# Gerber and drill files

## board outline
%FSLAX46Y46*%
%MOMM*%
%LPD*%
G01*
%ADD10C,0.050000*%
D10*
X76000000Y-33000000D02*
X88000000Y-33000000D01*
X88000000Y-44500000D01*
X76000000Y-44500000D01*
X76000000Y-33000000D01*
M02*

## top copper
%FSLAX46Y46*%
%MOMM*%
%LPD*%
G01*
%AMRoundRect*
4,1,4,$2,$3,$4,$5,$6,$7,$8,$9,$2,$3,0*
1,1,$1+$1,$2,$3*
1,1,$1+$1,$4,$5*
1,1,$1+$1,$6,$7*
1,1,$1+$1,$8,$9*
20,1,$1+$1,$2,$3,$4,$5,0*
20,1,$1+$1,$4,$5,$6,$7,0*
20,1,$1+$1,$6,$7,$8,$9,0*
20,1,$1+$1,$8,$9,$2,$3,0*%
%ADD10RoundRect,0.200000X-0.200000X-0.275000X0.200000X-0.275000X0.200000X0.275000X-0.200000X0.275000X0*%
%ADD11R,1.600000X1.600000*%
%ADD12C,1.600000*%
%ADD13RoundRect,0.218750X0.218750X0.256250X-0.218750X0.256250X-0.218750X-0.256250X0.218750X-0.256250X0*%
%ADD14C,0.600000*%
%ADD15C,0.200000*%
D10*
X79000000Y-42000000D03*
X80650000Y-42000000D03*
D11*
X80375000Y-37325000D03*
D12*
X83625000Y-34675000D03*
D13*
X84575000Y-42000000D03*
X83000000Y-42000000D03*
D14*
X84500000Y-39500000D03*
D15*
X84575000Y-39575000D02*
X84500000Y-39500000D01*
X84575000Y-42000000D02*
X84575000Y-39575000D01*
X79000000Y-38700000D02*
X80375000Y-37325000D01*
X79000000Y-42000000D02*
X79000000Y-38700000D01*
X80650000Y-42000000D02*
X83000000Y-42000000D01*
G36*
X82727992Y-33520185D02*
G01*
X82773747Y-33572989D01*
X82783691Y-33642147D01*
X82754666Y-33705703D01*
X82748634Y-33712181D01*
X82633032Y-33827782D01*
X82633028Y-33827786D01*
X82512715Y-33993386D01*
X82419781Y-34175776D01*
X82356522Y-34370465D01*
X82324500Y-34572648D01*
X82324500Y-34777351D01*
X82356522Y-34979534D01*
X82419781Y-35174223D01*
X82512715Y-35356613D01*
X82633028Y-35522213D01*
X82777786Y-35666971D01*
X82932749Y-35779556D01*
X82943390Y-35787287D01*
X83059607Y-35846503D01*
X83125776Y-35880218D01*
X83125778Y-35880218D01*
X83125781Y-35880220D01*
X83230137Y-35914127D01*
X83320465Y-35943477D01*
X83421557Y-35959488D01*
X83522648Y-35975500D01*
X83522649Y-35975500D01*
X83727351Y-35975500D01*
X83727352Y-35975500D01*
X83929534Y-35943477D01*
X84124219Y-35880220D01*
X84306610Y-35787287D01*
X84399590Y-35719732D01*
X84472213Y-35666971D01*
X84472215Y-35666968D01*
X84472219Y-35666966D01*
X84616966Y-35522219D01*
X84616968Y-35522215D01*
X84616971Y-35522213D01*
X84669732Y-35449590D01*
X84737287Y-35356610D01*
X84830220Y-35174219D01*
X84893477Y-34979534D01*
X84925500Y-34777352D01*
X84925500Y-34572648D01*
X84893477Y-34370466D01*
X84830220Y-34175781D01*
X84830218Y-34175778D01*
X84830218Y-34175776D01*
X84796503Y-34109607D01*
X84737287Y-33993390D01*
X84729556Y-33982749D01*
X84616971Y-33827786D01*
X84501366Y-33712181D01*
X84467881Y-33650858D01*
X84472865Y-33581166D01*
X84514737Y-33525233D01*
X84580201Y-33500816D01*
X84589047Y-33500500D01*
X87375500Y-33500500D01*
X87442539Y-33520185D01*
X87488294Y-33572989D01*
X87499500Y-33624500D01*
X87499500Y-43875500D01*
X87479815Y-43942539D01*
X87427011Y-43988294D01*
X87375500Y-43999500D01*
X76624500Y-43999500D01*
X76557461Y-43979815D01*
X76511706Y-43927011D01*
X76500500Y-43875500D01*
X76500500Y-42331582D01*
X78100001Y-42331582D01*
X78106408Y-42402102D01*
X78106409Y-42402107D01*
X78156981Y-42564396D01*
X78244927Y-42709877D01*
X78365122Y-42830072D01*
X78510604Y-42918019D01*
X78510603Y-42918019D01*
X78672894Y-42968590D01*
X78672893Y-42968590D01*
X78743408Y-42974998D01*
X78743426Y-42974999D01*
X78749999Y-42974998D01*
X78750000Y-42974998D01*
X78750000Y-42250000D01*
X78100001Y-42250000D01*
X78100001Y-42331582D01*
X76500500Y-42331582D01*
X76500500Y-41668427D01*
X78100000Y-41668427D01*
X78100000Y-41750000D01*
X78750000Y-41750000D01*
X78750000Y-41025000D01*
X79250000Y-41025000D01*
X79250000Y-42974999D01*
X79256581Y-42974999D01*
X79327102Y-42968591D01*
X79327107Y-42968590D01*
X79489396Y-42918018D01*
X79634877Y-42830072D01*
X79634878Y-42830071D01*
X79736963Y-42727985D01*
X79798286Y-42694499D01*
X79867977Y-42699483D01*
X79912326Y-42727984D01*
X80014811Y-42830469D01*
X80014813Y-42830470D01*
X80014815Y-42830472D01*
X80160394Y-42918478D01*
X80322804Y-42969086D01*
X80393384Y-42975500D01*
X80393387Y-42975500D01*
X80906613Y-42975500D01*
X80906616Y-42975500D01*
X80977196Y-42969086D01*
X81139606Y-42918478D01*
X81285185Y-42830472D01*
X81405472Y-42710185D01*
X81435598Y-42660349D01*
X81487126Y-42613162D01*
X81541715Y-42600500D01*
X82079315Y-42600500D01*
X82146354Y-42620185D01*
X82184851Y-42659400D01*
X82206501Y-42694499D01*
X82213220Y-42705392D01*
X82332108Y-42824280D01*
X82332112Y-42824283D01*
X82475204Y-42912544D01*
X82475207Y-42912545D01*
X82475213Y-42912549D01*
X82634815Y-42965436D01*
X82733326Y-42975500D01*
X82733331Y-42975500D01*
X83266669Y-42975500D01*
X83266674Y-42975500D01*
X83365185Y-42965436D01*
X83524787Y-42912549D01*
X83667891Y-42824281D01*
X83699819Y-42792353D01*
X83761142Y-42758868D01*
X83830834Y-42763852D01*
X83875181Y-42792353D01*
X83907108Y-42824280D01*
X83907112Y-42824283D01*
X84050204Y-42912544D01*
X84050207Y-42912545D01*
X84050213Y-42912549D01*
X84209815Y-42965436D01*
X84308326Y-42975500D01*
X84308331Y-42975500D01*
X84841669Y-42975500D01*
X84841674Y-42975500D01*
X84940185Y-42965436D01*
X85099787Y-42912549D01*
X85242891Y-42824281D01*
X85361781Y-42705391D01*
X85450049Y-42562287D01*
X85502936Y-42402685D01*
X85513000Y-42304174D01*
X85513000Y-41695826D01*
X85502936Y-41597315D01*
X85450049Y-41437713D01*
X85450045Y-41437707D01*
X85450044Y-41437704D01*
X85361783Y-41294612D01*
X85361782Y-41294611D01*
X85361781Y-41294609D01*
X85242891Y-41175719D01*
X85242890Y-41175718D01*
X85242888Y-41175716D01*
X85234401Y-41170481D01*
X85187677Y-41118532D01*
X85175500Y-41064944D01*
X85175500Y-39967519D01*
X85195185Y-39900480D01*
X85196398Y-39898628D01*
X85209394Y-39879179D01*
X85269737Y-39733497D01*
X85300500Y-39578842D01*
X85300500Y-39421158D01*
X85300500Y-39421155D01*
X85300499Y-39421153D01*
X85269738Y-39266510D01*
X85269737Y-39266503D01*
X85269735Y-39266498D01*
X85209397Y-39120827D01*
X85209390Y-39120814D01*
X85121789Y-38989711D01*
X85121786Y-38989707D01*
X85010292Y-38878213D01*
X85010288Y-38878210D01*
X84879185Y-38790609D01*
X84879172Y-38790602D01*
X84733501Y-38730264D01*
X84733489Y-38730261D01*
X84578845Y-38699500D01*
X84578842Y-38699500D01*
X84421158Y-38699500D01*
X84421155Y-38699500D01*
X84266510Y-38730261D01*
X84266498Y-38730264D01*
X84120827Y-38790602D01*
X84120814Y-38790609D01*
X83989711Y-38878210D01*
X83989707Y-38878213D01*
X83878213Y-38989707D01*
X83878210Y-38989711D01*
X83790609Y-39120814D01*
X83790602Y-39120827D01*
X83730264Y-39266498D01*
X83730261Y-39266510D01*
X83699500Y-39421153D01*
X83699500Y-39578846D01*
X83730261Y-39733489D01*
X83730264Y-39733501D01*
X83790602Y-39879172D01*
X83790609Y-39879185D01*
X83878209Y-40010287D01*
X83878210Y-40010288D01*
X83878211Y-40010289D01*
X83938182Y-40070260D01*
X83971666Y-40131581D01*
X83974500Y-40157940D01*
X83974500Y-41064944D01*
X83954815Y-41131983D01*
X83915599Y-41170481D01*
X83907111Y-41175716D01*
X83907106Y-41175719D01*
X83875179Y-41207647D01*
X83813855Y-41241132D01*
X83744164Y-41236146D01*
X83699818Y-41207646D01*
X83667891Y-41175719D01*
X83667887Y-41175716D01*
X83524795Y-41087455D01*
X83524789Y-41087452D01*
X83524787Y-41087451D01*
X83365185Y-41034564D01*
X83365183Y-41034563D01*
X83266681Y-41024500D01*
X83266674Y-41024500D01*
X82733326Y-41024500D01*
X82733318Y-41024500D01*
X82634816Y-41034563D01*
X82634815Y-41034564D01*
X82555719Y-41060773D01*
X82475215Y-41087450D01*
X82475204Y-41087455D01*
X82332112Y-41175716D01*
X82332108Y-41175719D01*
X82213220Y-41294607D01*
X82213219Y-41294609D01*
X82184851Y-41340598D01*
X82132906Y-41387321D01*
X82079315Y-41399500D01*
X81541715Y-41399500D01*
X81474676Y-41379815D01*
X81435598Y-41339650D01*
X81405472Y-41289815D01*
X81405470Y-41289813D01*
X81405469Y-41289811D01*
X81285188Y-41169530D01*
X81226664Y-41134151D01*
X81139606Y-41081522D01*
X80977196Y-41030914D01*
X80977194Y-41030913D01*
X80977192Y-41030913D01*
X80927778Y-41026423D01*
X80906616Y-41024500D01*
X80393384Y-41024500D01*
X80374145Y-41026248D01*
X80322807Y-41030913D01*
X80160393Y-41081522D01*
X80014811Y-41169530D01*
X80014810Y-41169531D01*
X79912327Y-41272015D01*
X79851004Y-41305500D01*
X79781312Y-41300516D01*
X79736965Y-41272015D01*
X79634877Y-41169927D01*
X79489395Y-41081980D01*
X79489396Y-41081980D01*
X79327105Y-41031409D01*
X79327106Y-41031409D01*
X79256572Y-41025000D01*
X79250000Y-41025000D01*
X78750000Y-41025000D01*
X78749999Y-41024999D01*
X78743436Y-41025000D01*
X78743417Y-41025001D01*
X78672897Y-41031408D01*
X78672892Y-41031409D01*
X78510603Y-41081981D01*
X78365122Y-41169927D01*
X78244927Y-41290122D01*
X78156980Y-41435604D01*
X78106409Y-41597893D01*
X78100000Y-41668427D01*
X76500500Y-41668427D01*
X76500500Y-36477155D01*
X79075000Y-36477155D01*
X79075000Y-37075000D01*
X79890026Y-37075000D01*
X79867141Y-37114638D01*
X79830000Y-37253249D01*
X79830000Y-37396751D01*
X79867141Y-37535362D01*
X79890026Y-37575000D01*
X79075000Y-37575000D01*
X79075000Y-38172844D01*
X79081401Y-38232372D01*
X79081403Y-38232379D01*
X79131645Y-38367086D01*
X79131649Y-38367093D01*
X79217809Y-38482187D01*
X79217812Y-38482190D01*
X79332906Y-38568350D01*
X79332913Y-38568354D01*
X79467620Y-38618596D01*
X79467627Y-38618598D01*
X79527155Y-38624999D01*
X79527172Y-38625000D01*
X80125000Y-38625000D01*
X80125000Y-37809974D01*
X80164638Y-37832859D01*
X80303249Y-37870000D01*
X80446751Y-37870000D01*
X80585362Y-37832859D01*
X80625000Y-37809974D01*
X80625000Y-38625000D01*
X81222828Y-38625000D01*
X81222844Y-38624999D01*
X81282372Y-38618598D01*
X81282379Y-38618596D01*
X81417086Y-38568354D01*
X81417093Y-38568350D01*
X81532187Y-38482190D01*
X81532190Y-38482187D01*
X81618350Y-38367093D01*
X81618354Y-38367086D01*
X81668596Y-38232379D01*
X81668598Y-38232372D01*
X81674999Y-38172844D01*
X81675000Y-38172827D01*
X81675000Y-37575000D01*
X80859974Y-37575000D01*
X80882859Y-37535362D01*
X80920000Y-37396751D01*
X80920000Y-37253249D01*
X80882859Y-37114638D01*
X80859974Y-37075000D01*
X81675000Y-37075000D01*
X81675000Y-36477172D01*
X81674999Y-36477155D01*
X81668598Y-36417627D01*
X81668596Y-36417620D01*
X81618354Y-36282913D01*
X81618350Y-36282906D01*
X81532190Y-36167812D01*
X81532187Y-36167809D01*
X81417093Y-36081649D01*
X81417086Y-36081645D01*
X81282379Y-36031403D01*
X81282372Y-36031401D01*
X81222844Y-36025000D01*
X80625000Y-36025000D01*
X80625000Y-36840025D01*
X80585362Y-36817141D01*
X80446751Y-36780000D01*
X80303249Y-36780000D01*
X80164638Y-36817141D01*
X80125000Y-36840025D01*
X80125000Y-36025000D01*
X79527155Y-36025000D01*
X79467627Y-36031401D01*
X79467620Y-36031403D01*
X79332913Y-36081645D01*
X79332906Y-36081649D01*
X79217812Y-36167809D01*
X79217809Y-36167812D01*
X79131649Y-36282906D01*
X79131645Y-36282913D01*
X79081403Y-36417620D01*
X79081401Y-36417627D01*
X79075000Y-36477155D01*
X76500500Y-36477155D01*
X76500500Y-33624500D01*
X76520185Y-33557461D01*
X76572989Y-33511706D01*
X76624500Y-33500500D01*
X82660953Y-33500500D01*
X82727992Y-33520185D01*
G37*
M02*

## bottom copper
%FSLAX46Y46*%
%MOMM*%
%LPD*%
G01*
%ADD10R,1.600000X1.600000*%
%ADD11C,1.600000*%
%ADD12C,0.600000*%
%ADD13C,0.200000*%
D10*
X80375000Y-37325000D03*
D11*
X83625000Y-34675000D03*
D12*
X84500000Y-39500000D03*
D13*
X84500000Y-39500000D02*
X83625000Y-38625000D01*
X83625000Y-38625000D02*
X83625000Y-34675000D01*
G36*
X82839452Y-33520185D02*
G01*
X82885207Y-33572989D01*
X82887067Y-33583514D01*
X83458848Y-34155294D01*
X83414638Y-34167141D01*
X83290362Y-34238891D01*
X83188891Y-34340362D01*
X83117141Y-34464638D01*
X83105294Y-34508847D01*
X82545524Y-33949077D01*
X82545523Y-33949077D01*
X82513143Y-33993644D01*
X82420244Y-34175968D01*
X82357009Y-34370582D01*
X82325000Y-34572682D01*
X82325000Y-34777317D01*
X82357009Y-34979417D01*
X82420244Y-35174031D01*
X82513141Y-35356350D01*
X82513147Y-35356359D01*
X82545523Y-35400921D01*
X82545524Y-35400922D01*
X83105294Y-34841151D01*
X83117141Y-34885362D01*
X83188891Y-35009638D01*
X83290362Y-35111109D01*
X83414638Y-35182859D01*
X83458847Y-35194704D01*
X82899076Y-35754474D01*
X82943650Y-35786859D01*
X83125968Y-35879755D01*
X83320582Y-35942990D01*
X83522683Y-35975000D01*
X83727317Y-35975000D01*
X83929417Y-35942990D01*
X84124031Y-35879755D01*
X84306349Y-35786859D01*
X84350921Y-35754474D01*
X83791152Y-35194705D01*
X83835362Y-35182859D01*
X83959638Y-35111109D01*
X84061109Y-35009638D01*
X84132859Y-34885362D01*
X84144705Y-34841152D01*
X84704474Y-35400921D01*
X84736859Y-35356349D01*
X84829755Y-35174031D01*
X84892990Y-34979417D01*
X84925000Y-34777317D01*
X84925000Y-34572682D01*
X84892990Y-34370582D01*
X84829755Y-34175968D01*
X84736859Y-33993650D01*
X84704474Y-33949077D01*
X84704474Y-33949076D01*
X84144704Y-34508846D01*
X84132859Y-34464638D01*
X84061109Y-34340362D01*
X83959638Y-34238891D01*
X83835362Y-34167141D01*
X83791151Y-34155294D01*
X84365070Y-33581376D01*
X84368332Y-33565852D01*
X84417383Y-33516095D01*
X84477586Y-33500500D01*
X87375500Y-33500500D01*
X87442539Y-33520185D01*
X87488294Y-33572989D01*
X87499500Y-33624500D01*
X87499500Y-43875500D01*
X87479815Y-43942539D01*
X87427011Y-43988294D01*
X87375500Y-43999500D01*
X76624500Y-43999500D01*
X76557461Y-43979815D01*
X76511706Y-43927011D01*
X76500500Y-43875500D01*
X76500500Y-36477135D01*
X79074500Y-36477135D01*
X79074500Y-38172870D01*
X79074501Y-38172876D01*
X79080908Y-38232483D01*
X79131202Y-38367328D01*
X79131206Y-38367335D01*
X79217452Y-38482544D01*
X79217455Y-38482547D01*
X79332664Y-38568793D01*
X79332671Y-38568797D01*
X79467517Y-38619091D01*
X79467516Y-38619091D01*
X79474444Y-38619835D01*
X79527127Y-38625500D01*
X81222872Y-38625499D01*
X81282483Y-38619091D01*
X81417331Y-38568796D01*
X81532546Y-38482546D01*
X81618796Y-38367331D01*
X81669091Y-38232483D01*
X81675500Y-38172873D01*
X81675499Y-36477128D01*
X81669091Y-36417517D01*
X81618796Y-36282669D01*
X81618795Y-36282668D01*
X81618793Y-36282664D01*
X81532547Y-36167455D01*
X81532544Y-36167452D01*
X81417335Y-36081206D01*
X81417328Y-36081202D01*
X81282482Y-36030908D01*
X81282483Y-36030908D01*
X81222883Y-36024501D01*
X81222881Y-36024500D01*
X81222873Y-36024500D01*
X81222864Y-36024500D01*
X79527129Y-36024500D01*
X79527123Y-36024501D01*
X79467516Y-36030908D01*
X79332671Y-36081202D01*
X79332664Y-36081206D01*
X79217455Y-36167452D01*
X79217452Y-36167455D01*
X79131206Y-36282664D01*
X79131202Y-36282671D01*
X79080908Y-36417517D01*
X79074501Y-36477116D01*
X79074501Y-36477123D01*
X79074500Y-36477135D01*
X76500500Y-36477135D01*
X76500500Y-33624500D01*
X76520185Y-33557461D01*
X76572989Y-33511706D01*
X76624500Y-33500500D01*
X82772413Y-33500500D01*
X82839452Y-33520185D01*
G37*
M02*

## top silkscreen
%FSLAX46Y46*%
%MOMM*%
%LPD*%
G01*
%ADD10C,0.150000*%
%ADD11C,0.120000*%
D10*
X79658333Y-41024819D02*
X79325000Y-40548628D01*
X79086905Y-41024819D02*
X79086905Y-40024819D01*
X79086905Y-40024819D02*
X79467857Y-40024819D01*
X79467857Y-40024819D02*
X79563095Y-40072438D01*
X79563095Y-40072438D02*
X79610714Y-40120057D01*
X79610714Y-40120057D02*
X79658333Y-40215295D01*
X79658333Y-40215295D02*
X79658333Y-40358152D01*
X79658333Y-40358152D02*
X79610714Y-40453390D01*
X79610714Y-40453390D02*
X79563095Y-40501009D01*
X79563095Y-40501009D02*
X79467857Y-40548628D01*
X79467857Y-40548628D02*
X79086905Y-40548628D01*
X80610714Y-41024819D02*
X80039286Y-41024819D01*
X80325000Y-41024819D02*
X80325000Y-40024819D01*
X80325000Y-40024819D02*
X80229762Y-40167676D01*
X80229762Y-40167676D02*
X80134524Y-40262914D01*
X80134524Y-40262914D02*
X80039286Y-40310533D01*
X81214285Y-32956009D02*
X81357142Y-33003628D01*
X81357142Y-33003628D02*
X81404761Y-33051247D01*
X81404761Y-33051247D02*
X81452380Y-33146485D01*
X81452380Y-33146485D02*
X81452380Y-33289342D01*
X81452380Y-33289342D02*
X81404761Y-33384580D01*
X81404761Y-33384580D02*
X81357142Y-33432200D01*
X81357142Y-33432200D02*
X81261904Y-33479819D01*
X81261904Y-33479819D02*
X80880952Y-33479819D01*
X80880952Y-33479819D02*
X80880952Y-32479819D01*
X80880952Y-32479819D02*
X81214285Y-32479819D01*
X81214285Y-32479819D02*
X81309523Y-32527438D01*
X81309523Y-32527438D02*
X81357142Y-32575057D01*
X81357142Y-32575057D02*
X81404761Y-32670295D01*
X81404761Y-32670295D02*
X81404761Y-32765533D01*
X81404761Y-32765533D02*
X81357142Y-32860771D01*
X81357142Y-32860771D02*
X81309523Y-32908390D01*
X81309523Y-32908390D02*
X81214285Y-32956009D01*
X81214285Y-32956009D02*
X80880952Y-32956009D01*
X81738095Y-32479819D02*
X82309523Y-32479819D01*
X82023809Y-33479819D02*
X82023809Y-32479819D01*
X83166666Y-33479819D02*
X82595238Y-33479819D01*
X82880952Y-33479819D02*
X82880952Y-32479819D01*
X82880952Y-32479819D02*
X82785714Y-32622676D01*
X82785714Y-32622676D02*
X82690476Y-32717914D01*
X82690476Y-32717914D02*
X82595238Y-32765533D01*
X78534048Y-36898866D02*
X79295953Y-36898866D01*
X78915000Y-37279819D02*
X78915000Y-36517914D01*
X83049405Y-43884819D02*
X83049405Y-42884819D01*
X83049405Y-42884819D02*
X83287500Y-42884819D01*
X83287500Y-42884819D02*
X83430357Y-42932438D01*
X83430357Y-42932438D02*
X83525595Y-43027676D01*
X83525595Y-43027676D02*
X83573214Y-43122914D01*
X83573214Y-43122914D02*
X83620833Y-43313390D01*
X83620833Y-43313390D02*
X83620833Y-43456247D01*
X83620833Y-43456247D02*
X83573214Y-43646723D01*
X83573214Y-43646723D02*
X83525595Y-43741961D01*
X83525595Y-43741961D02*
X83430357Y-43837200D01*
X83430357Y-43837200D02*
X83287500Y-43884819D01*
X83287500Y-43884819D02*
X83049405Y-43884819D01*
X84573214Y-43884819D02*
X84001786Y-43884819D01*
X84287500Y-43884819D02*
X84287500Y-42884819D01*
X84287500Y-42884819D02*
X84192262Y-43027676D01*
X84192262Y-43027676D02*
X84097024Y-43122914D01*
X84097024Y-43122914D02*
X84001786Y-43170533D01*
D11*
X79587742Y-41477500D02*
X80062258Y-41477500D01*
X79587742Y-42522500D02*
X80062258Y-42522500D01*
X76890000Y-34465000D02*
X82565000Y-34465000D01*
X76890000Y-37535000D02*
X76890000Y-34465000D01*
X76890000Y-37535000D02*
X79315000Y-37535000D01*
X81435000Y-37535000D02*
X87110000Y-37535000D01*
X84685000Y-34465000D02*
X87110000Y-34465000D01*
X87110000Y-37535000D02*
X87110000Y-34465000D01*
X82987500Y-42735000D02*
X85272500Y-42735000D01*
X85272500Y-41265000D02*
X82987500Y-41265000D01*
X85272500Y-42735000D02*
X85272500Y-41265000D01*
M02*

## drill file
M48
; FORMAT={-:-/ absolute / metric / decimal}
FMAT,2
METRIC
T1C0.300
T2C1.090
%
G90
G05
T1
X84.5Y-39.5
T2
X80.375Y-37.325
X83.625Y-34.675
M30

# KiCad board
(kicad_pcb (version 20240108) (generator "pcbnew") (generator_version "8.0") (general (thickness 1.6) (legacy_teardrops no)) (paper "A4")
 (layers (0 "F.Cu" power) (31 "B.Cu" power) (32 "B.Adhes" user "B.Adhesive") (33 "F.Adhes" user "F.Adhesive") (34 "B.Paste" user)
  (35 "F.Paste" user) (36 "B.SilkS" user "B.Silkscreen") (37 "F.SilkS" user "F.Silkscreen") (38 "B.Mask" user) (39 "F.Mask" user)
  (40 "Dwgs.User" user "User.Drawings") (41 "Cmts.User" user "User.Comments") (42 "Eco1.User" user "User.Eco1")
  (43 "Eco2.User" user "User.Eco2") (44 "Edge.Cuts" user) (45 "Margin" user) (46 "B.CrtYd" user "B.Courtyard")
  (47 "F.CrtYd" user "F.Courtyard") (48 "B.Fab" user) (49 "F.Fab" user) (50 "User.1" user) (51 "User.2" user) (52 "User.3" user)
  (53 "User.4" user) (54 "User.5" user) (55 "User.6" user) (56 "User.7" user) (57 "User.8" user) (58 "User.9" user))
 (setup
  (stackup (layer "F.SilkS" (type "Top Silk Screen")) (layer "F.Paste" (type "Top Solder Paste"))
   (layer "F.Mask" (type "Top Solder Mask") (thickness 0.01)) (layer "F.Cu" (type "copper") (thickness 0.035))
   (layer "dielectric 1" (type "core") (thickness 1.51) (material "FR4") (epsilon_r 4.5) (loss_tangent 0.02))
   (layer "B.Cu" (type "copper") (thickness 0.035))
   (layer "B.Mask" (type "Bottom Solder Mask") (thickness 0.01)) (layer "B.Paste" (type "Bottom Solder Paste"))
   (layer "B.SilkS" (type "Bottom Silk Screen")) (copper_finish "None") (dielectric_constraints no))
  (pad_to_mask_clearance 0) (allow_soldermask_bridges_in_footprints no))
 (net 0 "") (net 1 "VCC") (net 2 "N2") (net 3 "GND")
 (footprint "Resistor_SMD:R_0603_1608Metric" (layer "F.Cu") (at 79.825 42)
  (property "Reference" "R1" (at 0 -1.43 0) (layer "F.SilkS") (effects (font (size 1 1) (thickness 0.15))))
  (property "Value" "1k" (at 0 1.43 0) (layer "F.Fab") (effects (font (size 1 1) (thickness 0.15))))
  (fp_line (start -0.237258 -0.5225) (end 0.237258 -0.5225) (stroke (width 0.12) (type solid)) (layer "F.SilkS"))
  (fp_line (start -0.237258 0.5225) (end 0.237258 0.5225) (stroke (width 0.12) (type solid)) (layer "F.SilkS"))
  (pad "1" smd roundrect (at -0.825 0) (size 0.8 0.95) (layers "F.Cu" "F.Paste" "F.Mask") (roundrect_rratio 0.25) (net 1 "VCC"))
  (pad "2" smd roundrect (at 0.825 0) (size 0.8 0.95) (layers "F.Cu" "F.Paste" "F.Mask") (roundrect_rratio 0.25) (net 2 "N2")))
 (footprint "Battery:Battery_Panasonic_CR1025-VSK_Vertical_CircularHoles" (layer "F.Cu") (at 80.375 37.325)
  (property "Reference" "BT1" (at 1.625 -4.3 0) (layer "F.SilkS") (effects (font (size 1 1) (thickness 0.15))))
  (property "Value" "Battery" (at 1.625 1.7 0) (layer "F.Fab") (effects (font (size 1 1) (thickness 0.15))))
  (fp_line (start -3.485 -2.86) (end 2.19 -2.86) (stroke (width 0.12) (type solid)) (layer "F.SilkS"))
  (fp_line (start -3.485 0.21) (end -3.485 -2.86) (stroke (width 0.12) (type solid)) (layer "F.SilkS"))
  (fp_line (start -3.485 0.21) (end -1.06 0.21) (stroke (width 0.12) (type solid)) (layer "F.SilkS"))
  (fp_line (start 1.06 0.21) (end 6.735 0.21) (stroke (width 0.12) (type solid)) (layer "F.SilkS"))
  (fp_line (start 4.31 -2.86) (end 6.735 -2.86) (stroke (width 0.12) (type solid)) (layer "F.SilkS"))
  (fp_line (start 6.735 0.21) (end 6.735 -2.86) (stroke (width 0.12) (type solid)) (layer "F.SilkS"))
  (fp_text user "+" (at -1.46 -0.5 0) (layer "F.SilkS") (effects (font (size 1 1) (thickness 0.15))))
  (pad "1" thru_hole rect (at 0 0) (size 1.6 1.6) (drill 1.09) (layers "*.Cu" "*.Mask") (remove_unused_layers no) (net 1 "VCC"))
  (pad "2" thru_hole circle (at 3.25 -2.65) (size 1.6 1.6) (drill 1.09) (layers "*.Cu" "*.Mask") (remove_unused_layers no) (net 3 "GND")))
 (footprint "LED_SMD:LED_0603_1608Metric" (layer "F.Cu") (at 83.7875 42 180)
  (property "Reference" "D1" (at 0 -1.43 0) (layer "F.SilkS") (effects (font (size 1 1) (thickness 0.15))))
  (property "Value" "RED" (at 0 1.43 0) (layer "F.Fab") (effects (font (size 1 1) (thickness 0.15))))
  (fp_line (start 0.8 -0.735) (end -1.485 -0.735) (stroke (width 0.12) (type solid)) (layer "F.SilkS"))
  (fp_line (start -1.485 0.735) (end 0.8 0.735) (stroke (width 0.12) (type solid)) (layer "F.SilkS"))
  (fp_line (start -1.485 -0.735) (end -1.485 0.735) (stroke (width 0.12) (type solid)) (layer "F.SilkS"))
  (pad "1" smd roundrect (at -0.7875 0 180) (size 0.875 0.95) (layers "F.Cu" "F.Paste" "F.Mask") (roundrect_rratio 0.25) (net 3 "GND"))
  (pad "2" smd roundrect (at 0.7875 0 180) (size 0.875 0.95) (layers "F.Cu" "F.Paste" "F.Mask") (roundrect_rratio 0.25) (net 2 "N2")))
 (gr_rect (start 76 33) (end 88 44.5) (stroke (width 0.05) (type default)) (fill none) (layer "Edge.Cuts"))
 (segment (start 84.575 39.575) (end 84.5 39.5) (width 0.2) (layer "F.Cu") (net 3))
 (segment (start 84.575 42) (end 84.575 39.575) (width 0.2) (layer "F.Cu") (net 3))
 (via (at 84.5 39.5) (size 0.6) (drill 0.3) (layers "F.Cu" "B.Cu") (free yes) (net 3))
 (segment (start 84.5 39.5) (end 83.625 38.625) (width 0.2) (layer "B.Cu") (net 3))
 (segment (start 83.625 38.625) (end 83.625 34.675) (width 0.2) (layer "B.Cu") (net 3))
 (segment (start 79 38.7) (end 80.375 37.325) (width 0.2) (layer "F.Cu") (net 1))
 (segment (start 79 42) (end 79 38.7) (width 0.2) (layer "F.Cu") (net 1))
 (segment (start 80.65 42) (end 83 42) (width 0.2) (layer "F.Cu") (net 2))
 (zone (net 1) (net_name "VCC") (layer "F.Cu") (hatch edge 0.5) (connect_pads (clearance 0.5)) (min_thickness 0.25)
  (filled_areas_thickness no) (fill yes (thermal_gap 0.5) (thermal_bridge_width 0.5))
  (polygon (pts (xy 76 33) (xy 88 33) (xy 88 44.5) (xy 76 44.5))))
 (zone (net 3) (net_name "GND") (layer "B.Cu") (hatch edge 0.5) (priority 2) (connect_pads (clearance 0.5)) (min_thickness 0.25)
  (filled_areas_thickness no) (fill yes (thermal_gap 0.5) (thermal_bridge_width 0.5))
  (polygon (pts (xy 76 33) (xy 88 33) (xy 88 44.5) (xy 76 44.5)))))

